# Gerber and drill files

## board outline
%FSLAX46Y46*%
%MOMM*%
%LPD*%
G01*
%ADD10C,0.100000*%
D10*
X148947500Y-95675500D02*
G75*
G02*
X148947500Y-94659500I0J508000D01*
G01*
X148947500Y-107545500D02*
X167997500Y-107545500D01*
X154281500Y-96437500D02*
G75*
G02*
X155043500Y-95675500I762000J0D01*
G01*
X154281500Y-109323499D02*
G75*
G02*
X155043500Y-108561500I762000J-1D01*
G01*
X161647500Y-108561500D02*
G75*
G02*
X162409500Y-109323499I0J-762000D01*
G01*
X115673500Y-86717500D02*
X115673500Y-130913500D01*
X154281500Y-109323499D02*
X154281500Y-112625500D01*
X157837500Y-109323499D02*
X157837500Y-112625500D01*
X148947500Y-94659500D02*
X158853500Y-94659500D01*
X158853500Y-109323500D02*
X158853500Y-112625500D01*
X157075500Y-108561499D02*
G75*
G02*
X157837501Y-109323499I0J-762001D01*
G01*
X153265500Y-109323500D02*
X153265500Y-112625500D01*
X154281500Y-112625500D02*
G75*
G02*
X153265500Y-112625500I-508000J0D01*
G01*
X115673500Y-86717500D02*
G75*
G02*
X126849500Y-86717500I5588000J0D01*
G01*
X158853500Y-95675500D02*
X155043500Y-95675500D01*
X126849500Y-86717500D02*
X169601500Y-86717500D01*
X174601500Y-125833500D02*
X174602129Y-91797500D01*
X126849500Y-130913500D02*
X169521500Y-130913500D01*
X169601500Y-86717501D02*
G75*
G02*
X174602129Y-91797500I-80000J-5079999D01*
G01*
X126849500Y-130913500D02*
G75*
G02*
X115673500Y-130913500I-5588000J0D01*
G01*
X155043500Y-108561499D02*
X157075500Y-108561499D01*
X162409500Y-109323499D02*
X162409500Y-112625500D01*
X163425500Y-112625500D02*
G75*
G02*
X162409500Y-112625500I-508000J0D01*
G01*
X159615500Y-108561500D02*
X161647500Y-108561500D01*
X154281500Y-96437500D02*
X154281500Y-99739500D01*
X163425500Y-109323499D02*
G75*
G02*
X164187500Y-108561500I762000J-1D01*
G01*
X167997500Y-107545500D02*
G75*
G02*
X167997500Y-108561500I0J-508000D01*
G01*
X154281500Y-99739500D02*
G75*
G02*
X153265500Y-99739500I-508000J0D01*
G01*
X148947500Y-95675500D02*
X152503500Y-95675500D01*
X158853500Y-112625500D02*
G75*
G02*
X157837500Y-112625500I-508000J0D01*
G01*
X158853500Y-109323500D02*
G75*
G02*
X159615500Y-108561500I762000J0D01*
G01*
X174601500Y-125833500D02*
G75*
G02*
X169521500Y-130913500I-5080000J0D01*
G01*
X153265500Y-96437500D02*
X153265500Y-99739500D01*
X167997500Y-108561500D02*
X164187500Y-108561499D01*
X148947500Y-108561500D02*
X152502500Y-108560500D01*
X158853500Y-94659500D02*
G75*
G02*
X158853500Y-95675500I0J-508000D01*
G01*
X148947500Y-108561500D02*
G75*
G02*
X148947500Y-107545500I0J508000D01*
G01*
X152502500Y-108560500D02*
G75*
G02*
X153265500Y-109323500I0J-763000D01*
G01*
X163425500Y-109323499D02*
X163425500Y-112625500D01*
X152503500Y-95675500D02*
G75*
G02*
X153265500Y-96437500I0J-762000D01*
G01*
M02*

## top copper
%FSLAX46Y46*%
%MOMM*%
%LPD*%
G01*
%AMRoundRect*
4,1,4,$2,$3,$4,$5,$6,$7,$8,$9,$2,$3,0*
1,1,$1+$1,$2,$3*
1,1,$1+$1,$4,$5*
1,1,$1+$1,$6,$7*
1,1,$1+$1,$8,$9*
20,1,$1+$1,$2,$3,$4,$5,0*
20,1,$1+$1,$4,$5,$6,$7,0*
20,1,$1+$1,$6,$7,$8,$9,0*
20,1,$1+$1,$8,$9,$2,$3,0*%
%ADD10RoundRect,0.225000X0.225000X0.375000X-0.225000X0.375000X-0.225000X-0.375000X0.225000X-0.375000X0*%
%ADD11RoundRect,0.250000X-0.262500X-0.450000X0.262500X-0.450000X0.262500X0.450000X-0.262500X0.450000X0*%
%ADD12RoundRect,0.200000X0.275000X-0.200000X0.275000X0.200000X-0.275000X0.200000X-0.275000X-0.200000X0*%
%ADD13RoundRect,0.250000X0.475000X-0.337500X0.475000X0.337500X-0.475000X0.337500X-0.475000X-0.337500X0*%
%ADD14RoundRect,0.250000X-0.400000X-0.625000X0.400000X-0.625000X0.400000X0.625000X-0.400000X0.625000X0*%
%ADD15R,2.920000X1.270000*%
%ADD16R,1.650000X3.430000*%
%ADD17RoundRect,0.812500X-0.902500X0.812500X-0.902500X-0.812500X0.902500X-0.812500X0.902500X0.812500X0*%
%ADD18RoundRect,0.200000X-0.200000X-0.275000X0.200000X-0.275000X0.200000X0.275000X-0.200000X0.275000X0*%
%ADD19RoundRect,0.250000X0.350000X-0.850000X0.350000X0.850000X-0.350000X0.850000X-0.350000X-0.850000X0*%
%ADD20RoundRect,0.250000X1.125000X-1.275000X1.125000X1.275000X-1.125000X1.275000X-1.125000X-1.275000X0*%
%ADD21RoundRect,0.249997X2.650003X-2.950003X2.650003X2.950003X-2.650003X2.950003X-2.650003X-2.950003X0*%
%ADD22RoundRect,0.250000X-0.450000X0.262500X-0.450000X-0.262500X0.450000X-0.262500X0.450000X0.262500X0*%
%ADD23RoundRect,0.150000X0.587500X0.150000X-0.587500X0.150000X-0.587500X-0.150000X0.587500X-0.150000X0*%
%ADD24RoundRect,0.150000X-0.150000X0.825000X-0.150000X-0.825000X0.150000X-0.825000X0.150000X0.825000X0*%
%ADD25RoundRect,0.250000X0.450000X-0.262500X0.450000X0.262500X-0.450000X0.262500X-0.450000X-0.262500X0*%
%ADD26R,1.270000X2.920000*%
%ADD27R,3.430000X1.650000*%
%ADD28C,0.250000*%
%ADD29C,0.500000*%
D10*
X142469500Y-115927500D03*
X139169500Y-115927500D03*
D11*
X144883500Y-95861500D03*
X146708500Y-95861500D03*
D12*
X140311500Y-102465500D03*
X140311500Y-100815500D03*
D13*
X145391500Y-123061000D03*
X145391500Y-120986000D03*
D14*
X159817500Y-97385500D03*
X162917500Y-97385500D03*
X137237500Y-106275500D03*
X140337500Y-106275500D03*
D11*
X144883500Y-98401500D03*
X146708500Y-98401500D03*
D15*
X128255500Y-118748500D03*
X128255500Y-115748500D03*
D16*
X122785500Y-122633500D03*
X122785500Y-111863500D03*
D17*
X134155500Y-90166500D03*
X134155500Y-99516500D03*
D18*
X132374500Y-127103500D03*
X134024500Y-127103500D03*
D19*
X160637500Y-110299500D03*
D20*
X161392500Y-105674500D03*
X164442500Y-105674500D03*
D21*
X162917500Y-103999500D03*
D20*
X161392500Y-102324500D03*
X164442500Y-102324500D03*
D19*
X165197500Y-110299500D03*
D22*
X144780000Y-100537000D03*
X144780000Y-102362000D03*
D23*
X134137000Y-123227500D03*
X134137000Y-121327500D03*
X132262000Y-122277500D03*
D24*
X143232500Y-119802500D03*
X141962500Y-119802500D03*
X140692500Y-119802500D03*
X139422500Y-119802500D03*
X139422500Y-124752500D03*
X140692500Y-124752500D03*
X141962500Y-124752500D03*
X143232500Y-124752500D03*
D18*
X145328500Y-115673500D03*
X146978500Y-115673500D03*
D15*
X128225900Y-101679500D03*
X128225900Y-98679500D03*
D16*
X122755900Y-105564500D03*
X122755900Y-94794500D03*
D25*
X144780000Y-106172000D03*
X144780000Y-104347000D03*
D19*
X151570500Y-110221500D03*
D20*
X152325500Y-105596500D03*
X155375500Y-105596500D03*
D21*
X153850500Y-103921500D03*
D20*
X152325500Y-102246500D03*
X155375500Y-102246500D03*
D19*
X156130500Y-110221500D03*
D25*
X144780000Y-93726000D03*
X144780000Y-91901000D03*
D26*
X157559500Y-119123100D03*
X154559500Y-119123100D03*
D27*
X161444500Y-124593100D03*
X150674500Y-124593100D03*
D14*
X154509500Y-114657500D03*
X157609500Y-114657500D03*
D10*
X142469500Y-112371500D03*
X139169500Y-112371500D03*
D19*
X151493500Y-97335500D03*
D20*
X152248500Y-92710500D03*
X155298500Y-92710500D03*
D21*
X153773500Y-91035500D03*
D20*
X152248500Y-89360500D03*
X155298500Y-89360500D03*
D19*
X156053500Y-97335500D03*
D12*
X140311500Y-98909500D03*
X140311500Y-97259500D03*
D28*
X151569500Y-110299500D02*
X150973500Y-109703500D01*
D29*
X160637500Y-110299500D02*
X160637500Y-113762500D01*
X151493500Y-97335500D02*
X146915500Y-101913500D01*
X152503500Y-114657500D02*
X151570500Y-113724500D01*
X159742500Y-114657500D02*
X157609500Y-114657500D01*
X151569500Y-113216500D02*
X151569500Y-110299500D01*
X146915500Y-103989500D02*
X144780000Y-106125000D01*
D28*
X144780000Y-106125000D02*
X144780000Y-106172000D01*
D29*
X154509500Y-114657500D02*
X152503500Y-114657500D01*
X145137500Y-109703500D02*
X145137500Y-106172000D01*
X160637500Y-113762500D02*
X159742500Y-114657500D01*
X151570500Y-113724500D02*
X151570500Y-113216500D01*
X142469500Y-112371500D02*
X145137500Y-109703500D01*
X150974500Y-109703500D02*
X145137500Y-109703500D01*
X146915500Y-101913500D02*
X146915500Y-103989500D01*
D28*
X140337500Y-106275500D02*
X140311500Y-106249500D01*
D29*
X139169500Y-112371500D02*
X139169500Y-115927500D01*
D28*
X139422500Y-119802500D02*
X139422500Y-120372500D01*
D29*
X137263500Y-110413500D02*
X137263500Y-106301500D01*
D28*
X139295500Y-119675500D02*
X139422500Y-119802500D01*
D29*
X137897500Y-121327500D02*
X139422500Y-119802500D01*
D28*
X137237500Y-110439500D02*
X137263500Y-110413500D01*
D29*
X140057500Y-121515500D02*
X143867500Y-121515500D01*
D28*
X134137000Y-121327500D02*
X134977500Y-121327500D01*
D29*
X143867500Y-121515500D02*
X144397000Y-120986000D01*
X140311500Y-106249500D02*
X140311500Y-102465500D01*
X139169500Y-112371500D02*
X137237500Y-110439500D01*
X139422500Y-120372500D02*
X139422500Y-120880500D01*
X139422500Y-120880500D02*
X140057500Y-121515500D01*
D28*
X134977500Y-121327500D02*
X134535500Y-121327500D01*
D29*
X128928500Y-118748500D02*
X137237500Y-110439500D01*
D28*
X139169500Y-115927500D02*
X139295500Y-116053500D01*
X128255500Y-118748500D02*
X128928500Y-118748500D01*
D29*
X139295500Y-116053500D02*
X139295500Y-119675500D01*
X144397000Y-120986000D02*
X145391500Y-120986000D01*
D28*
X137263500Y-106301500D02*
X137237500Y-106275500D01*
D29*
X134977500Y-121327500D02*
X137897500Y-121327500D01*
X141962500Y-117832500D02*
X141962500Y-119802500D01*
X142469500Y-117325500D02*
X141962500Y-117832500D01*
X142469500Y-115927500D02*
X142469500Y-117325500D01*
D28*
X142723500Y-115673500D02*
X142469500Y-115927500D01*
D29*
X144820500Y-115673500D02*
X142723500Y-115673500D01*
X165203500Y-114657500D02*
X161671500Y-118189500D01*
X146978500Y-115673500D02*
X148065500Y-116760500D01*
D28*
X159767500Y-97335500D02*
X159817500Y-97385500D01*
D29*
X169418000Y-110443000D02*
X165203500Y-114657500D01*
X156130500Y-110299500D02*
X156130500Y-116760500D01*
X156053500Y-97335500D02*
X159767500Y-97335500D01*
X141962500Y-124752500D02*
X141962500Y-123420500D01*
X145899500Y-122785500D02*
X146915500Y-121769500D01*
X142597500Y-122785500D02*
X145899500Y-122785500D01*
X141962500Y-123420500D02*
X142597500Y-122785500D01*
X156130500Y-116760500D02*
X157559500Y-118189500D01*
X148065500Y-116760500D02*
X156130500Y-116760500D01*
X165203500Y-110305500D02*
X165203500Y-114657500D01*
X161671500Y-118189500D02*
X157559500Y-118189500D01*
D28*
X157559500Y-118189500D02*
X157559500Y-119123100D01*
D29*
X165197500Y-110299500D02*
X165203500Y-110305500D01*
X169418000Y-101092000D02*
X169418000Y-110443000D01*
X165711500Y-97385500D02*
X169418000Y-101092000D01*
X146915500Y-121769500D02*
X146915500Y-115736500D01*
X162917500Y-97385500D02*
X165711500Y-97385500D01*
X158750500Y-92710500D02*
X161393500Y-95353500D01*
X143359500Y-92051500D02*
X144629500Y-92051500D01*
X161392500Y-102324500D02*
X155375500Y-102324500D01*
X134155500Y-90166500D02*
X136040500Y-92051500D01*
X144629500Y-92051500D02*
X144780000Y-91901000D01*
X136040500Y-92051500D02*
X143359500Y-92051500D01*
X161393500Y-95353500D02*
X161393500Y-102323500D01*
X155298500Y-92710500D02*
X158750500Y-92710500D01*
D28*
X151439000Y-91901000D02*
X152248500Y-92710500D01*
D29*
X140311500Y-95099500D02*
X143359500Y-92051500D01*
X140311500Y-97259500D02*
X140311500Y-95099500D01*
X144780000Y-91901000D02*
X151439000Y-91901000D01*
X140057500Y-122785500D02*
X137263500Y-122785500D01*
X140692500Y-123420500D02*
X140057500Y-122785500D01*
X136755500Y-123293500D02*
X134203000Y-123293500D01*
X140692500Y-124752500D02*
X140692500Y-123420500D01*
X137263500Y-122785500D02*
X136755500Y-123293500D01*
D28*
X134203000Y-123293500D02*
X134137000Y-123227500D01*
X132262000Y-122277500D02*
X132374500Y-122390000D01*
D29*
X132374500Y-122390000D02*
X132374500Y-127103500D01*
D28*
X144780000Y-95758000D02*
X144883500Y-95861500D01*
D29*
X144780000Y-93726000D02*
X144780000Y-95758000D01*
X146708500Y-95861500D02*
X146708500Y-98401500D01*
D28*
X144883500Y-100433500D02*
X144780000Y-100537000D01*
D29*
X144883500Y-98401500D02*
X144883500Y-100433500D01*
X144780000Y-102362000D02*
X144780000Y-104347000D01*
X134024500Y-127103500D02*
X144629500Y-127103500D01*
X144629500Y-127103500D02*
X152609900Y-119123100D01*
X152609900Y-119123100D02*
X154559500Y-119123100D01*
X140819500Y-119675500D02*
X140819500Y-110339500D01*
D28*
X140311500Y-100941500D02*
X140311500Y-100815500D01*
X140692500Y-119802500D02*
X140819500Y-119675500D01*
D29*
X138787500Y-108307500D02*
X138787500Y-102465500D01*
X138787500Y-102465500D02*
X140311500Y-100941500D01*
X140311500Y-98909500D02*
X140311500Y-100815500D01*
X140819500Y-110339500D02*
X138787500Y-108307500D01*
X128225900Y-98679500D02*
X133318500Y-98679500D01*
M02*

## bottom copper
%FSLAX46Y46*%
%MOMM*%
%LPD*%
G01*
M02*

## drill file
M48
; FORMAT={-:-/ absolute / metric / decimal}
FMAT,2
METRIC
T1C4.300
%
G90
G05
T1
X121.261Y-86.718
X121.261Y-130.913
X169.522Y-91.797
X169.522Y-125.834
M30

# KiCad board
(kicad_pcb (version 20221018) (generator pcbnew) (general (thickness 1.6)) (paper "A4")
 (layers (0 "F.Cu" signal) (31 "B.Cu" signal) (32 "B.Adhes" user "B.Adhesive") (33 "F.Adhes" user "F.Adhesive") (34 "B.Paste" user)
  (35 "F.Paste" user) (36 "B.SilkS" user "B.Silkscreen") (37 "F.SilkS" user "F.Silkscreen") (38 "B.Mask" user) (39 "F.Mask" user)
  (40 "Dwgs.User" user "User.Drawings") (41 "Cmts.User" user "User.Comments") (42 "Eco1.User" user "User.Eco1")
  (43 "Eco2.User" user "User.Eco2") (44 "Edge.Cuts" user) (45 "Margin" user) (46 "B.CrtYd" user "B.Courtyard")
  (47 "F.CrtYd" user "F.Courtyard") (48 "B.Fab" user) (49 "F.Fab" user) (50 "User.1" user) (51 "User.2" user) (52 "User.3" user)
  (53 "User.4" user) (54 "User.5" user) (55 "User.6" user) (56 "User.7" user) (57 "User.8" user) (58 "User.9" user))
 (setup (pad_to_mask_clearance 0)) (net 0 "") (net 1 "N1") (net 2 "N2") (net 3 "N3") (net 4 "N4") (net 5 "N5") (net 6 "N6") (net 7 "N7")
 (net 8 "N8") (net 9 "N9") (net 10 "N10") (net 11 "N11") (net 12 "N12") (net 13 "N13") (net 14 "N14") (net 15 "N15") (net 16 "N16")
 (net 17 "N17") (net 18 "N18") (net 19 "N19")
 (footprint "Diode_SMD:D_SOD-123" (layer "F.Cu") (at 140.8195 115.9275 180)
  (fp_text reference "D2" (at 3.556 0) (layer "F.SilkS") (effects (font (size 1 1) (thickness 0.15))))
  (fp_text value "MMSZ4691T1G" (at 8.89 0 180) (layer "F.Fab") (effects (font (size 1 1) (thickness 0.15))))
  (pad "1" smd roundrect (at -1.65 0 180) (size 0.9 1.2) (layers "F.Cu" "F.Paste" "F.Mask") (roundrect_rratio 0.25) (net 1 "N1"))
  (pad "2" smd roundrect (at 1.65 0 180) (size 0.9 1.2) (layers "F.Cu" "F.Paste" "F.Mask") (roundrect_rratio 0.25) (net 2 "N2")))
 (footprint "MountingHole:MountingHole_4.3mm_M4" (layer "F.Cu") (at 169.5215 91.7975)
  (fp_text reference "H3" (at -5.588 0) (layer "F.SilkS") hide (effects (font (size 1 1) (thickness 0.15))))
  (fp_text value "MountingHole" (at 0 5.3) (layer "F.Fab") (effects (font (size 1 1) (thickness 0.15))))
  (pad "" np_thru_hole circle (at 0 0) (size 4.3 4.3) (drill 4.3) (layers "*.Cu" "*.Mask")))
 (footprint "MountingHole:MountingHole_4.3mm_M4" (layer "F.Cu") (at 121.2615 130.9135)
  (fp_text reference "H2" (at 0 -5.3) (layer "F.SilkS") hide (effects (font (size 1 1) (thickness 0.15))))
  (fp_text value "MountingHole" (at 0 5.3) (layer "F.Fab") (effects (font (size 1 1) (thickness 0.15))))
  (pad "" np_thru_hole circle (at 0 0) (size 4.3 4.3) (drill 4.3) (layers "*.Cu" "*.Mask")))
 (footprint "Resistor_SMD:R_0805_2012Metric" (layer "F.Cu") (at 145.796 95.8615)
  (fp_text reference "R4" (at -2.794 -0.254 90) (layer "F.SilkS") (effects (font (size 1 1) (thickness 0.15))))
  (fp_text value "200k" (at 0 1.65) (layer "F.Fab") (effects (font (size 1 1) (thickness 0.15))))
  (pad "1" smd roundrect (at -0.9125 0) (size 1.025 1.4) (layers "F.Cu" "F.Paste" "F.Mask") (roundrect_rratio 0.243902) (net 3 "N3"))
  (pad "2" smd roundrect (at 0.9125 0) (size 1.025 1.4) (layers "F.Cu" "F.Paste" "F.Mask") (roundrect_rratio 0.243902) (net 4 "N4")))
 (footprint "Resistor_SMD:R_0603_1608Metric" (layer "F.Cu") (at 140.3115 101.6405 90)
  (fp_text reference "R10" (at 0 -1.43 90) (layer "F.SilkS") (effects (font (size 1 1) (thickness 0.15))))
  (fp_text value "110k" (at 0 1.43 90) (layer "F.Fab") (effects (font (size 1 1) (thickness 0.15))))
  (pad "1" smd roundrect (at -0.825 0 90) (size 0.8 0.95) (layers "F.Cu" "F.Paste" "F.Mask") (roundrect_rratio 0.25) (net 2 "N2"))
  (pad "2" smd roundrect (at 0.825 0 90) (size 0.8 0.95) (layers "F.Cu" "F.Paste" "F.Mask") (roundrect_rratio 0.25) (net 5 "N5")))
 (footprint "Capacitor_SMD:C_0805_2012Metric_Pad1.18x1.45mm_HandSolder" (layer "F.Cu") (at 145.3915 122.0235 90)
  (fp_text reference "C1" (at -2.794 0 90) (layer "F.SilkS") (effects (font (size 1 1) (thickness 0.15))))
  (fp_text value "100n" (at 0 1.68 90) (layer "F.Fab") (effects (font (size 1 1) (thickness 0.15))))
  (pad "1" smd roundrect (at -1.0375 0 90) (size 1.175 1.45) (layers "F.Cu" "F.Paste" "F.Mask") (roundrect_rratio 0.212766) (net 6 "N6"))
  (pad "2" smd roundrect (at 1.0375 0 90) (size 1.175 1.45) (layers "F.Cu" "F.Paste" "F.Mask") (roundrect_rratio 0.212766) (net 2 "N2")))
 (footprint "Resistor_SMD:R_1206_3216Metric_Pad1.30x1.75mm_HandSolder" (layer "F.Cu") (at 161.3675 97.3855)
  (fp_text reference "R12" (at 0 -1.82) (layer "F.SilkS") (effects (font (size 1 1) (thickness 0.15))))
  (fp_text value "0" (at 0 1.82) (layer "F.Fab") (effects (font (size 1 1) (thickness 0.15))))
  (pad "1" smd roundrect (at -1.55 0) (size 1.3 1.75) (layers "F.Cu" "F.Paste" "F.Mask") (roundrect_rratio 0.192308) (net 6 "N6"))
  (pad "2" smd roundrect (at 1.55 0) (size 1.3 1.75) (layers "F.Cu" "F.Paste" "F.Mask") (roundrect_rratio 0.192308) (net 6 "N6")))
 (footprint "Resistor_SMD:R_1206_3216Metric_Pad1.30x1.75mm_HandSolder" (layer "F.Cu") (at 138.7875 106.2755)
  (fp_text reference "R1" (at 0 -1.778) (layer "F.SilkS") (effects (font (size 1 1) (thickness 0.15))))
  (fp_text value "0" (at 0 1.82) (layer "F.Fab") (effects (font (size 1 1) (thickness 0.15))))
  (pad "1" smd roundrect (at -1.55 0) (size 1.3 1.75) (layers "F.Cu" "F.Paste" "F.Mask") (roundrect_rratio 0.192308) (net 2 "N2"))
  (pad "2" smd roundrect (at 1.55 0) (size 1.3 1.75) (layers "F.Cu" "F.Paste" "F.Mask") (roundrect_rratio 0.192308) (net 2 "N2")))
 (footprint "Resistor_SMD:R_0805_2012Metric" (layer "F.Cu") (at 145.796 98.4015)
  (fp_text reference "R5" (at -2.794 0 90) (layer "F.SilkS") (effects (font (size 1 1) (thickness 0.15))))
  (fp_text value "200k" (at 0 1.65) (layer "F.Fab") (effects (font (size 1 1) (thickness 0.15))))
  (pad "1" smd roundrect (at -0.9125 0) (size 1.025 1.4) (layers "F.Cu" "F.Paste" "F.Mask") (roundrect_rratio 0.243902) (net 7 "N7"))
  (pad "2" smd roundrect (at 0.9125 0) (size 1.025 1.4) (layers "F.Cu" "F.Paste" "F.Mask") (roundrect_rratio 0.243902) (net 4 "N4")))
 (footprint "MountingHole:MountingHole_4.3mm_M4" (layer "F.Cu") (at 169.5215 125.8335)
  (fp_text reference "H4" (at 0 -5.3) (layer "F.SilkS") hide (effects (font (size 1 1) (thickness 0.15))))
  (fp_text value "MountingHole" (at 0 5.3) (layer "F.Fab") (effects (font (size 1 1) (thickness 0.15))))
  (pad "" np_thru_hole circle (at 0 0) (size 4.3 4.3) (drill 4.3) (layers "*.Cu" "*.Mask")))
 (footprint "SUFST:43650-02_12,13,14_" (layer "F.Cu") (at 128.2555 117.2485 -90)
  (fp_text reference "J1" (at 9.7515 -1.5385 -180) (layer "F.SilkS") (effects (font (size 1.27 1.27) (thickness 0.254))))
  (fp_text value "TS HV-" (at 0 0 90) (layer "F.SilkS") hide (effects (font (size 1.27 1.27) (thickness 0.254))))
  (pad "1" smd rect (at 1.5 0 270) (size 1.27 2.92) (layers "F.Cu" "F.Paste" "F.Mask") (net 2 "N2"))
  (pad "2" smd rect (at -1.5 0 270) (size 1.27 2.92) (layers "F.Cu" "F.Paste" "F.Mask") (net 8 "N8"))
  (pad "3" smd rect (at 5.385 5.47) (size 1.65 3.43) (layers "F.Cu" "F.Paste" "F.Mask"))
  (pad "4" smd rect (at -5.385 5.47) (size 1.65 3.43) (layers "F.Cu" "F.Paste" "F.Mask")))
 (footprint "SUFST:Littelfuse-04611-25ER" (layer "F.Cu") (at 134.2155 94.5915 -90)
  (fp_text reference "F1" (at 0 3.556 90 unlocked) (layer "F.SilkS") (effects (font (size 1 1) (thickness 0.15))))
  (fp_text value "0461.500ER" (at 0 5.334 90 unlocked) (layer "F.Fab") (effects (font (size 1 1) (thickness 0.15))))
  (pad "1" smd roundrect (at -4.425 0.06 270) (size 3.25 3.43) (layers "F.Cu" "F.Paste" "F.Mask") (roundrect_rratio 0.25) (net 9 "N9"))
  (pad "2" smd roundrect (at 4.925 0.06 270) (size 3.25 3.43) (layers "F.Cu" "F.Paste" "F.Mask") (roundrect_rratio 0.25) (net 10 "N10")))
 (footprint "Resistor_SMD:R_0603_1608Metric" (layer "F.Cu") (at 133.1995 127.1035)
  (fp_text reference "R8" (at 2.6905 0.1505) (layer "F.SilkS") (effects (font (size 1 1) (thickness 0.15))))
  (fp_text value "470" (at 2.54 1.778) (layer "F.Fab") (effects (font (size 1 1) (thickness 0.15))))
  (pad "1" smd roundrect (at -0.825 0) (size 0.8 0.95) (layers "F.Cu" "F.Paste" "F.Mask") (roundrect_rratio 0.25) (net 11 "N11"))
  (pad "2" smd roundrect (at 0.825 0) (size 0.8 0.95) (layers "F.Cu" "F.Paste" "F.Mask") (roundrect_rratio 0.25) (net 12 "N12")))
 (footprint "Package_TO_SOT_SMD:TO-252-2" (layer "F.Cu") (at 162.9175 105.2595 90)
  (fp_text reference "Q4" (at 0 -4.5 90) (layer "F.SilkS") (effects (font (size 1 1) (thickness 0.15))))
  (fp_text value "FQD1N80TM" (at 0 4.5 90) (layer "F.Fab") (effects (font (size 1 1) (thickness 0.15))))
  (pad "1" smd roundrect (at -5.04 -2.28 90) (size 2.2 1.2) (layers "F.Cu" "F.Paste" "F.Mask") (roundrect_rratio 0.208333) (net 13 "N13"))
  (pad "2" smd roundrect (at -0.415 -1.525 90) (size 3.05 2.75) (layers "F.Cu" "F.Paste") (roundrect_rratio 0.090909) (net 9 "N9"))
  (pad "2" smd roundrect (at -0.415 1.525 90) (size 3.05 2.75) (layers "F.Cu" "F.Paste") (roundrect_rratio 0.090909) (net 9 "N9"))
  (pad "2" smd roundrect (at 1.26 0 90) (size 6.4 5.8) (layers "F.Cu" "F.Mask") (roundrect_rratio 0.043103) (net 9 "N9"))
  (pad "2" smd roundrect (at 2.935 -1.525 90) (size 3.05 2.75) (layers "F.Cu" "F.Paste") (roundrect_rratio 0.090909) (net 9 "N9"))
  (pad "2" smd roundrect (at 2.935 1.525 90) (size 3.05 2.75) (layers "F.Cu" "F.Paste") (roundrect_rratio 0.090909) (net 9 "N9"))
  (pad "3" smd roundrect (at -5.04 2.28 90) (size 2.2 1.2) (layers "F.Cu" "F.Paste" "F.Mask") (roundrect_rratio 0.208333) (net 6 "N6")))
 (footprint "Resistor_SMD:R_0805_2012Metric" (layer "F.Cu") (at 144.78 101.4495 -90)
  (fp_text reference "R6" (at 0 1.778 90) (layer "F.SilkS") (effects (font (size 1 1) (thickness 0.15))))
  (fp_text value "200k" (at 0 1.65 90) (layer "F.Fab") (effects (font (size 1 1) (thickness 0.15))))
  (pad "1" smd roundrect (at -0.9125 0 270) (size 1.025 1.4) (layers "F.Cu" "F.Paste" "F.Mask") (roundrect_rratio 0.243902) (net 7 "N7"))
  (pad "2" smd roundrect (at 0.9125 0 270) (size 1.025 1.4) (layers "F.Cu" "F.Paste" "F.Mask") (roundrect_rratio 0.243902) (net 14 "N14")))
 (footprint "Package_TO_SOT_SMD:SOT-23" (layer "F.Cu") (at 133.1995 122.2775 180)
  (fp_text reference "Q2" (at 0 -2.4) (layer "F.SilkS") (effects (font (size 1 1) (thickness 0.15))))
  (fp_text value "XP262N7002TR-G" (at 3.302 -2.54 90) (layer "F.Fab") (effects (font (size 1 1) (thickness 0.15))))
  (pad "1" smd roundrect (at -0.9375 -0.95 180) (size 1.475 0.6) (layers "F.Cu" "F.Paste" "F.Mask") (roundrect_rratio 0.25) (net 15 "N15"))
  (pad "2" smd roundrect (at -0.9375 0.95 180) (size 1.475 0.6) (layers "F.Cu" "F.Paste" "F.Mask") (roundrect_rratio 0.25) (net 2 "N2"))
  (pad "3" smd roundrect (at 0.9375 0 180) (size 1.475 0.6) (layers "F.Cu" "F.Paste" "F.Mask") (roundrect_rratio 0.25) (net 11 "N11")))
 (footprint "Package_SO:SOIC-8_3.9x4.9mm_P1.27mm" (layer "F.Cu") (at 141.3275 122.2775 -90)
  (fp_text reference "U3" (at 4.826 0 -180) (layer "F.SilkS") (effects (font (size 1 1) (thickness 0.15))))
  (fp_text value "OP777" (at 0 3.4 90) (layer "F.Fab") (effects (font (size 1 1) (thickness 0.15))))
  (pad "1" smd roundrect (at -2.475 -1.905 270) (size 1.95 0.6) (layers "F.Cu" "F.Paste" "F.Mask") (roundrect_rratio 0.25) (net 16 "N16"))
  (pad "2" smd roundrect (at -2.475 -0.635 270) (size 1.95 0.6) (layers "F.Cu" "F.Paste" "F.Mask") (roundrect_rratio 0.25) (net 1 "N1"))
  (pad "3" smd roundrect (at -2.475 0.635 270) (size 1.95 0.6) (layers "F.Cu" "F.Paste" "F.Mask") (roundrect_rratio 0.25) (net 5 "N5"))
  (pad "4" smd roundrect (at -2.475 1.905 270) (size 1.95 0.6) (layers "F.Cu" "F.Paste" "F.Mask") (roundrect_rratio 0.25) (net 2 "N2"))
  (pad "5" smd roundrect (at 2.475 1.905 270) (size 1.95 0.6) (layers "F.Cu" "F.Paste" "F.Mask") (roundrect_rratio 0.25) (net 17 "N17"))
  (pad "6" smd roundrect (at 2.475 0.635 270) (size 1.95 0.6) (layers "F.Cu" "F.Paste" "F.Mask") (roundrect_rratio 0.25) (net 15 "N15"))
  (pad "7" smd roundrect (at 2.475 -0.635 270) (size 1.95 0.6) (layers "F.Cu" "F.Paste" "F.Mask") (roundrect_rratio 0.25) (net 6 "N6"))
  (pad "8" smd roundrect (at 2.475 -1.905 270) (size 1.95 0.6) (layers "F.Cu" "F.Paste" "F.Mask") (roundrect_rratio 0.25) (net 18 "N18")))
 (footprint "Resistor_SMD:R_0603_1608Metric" (layer "F.Cu") (at 146.1535 115.6735)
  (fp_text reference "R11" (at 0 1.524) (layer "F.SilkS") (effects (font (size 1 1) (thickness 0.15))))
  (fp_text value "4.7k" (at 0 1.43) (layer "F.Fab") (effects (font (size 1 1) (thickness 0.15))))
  (pad "1" smd roundrect (at -0.825 0) (size 0.8 0.95) (layers "F.Cu" "F.Paste" "F.Mask") (roundrect_rratio 0.25) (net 1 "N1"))
  (pad "2" smd roundrect (at 0.825 0) (size 0.8 0.95) (layers "F.Cu" "F.Paste" "F.Mask") (roundrect_rratio 0.25) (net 6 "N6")))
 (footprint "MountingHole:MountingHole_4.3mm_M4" (layer "F.Cu") (at 121.2615 86.7175)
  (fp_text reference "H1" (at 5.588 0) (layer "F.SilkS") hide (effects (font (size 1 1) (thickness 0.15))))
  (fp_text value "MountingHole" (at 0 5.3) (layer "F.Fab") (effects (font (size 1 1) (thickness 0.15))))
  (pad "" np_thru_hole circle (at 0 0) (size 4.3 4.3) (drill 4.3) (layers "*.Cu" "*.Mask")))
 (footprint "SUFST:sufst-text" (layer "F.Cu") (at 170.5375 109.0695 90)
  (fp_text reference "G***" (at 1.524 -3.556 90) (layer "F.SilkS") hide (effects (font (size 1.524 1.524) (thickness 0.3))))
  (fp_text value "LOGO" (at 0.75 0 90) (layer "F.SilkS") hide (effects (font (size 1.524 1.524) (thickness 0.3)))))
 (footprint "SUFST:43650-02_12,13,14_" (layer "F.Cu") (at 128.2259 100.1795 -90)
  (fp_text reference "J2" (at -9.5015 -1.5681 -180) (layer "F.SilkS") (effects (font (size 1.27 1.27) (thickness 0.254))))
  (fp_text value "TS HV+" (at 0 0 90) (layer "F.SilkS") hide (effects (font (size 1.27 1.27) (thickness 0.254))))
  (pad "1" smd rect (at 1.5 0 270) (size 1.27 2.92) (layers "F.Cu" "F.Paste" "F.Mask") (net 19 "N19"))
  (pad "2" smd rect (at -1.5 0 270) (size 1.27 2.92) (layers "F.Cu" "F.Paste" "F.Mask") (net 10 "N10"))
  (pad "3" smd rect (at 5.385 5.47) (size 1.65 3.43) (layers "F.Cu" "F.Paste" "F.Mask"))
  (pad "4" smd rect (at -5.385 5.47) (size 1.65 3.43) (layers "F.Cu" "F.Paste" "F.Mask")))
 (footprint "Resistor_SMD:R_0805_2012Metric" (layer "F.Cu") (at 144.78 105.2595 90)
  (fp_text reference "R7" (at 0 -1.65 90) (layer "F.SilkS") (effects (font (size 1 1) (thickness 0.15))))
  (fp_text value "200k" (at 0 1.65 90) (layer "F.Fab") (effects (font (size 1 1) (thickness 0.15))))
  (pad "1" smd roundrect (at -0.9125 0 90) (size 1.025 1.4) (layers "F.Cu" "F.Paste" "F.Mask") (roundrect_rratio 0.243902) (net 13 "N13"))
  (pad "2" smd roundrect (at 0.9125 0 90) (size 1.025 1.4) (layers "F.Cu" "F.Paste" "F.Mask") (roundrect_rratio 0.243902) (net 14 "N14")))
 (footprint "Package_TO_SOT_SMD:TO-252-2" (layer "F.Cu") (at 153.8505 105.1815 90)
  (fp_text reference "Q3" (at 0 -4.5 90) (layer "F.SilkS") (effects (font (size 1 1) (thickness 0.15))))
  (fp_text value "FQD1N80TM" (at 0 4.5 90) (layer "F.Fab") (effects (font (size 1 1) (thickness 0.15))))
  (pad "1" smd roundrect (at -5.04 -2.28 90) (size 2.2 1.2) (layers "F.Cu" "F.Paste" "F.Mask") (roundrect_rratio 0.208333) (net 13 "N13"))
  (pad "2" smd roundrect (at -0.415 -1.525 90) (size 3.05 2.75) (layers "F.Cu" "F.Paste") (roundrect_rratio 0.090909) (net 9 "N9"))
  (pad "2" smd roundrect (at -0.415 1.525 90) (size 3.05 2.75) (layers "F.Cu" "F.Paste") (roundrect_rratio 0.090909) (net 9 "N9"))
  (pad "2" smd roundrect (at 1.26 0 90) (size 6.4 5.8) (layers "F.Cu" "F.Mask") (roundrect_rratio 0.043103) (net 9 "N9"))
  (pad "2" smd roundrect (at 2.935 -1.525 90) (size 3.05 2.75) (layers "F.Cu" "F.Paste") (roundrect_rratio 0.090909) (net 9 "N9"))
  (pad "2" smd roundrect (at 2.935 1.525 90) (size 3.05 2.75) (layers "F.Cu" "F.Paste") (roundrect_rratio 0.090909) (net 9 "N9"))
  (pad "3" smd roundrect (at -5.04 2.28 90) (size 2.2 1.2) (layers "F.Cu" "F.Paste" "F.Mask") (roundrect_rratio 0.208333) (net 6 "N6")))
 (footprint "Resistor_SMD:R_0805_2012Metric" (layer "F.Cu") (at 144.78 92.8135 90)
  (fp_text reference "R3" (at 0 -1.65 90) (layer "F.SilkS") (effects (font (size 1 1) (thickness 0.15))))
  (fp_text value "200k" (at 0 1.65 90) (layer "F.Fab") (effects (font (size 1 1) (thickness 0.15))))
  (pad "1" smd roundrect (at -0.9125 0 90) (size 1.025 1.4) (layers "F.Cu" "F.Paste" "F.Mask") (roundrect_rratio 0.243902) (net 3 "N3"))
  (pad "2" smd roundrect (at 0.9125 0 90) (size 1.025 1.4) (layers "F.Cu" "F.Paste" "F.Mask") (roundrect_rratio 0.243902) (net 9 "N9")))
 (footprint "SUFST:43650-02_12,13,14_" (layer "F.Cu") (at 156.0595 119.1231)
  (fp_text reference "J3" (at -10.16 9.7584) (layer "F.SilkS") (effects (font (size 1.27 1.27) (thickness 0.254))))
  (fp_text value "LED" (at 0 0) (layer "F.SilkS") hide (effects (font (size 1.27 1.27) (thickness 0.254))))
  (pad "1" smd rect (at 1.5 0) (size 1.27 2.92) (layers "F.Cu" "F.Paste" "F.Mask") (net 6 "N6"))
  (pad "2" smd rect (at -1.5 0) (size 1.27 2.92) (layers "F.Cu" "F.Paste" "F.Mask") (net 12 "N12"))
  (pad "3" smd rect (at 5.385 5.47 90) (size 1.65 3.43) (layers "F.Cu" "F.Paste" "F.Mask"))
  (pad "4" smd rect (at -5.385 5.47 90) (size 1.65 3.43) (layers "F.Cu" "F.Paste" "F.Mask")))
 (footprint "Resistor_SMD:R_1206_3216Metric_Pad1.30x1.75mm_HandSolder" (layer "F.Cu") (at 156.0595 114.6575)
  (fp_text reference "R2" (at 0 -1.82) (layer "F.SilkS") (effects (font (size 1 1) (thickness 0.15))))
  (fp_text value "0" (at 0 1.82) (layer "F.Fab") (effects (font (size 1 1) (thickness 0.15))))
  (pad "1" smd roundrect (at -1.55 0) (size 1.3 1.75) (layers "F.Cu" "F.Paste" "F.Mask") (roundrect_rratio 0.192308) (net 13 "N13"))
  (pad "2" smd roundrect (at 1.55 0) (size 1.3 1.75) (layers "F.Cu" "F.Paste" "F.Mask") (roundrect_rratio 0.192308) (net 13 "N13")))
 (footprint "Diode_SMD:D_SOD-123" (layer "F.Cu") (at 140.8195 112.3715 180)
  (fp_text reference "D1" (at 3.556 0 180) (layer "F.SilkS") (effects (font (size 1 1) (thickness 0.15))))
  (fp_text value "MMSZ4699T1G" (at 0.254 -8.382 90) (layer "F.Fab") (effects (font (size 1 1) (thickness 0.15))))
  (pad "1" smd roundrect (at -1.65 0 180) (size 0.9 1.2) (layers "F.Cu" "F.Paste" "F.Mask") (roundrect_rratio 0.25) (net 13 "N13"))
  (pad "2" smd roundrect (at 1.65 0 180) (size 0.9 1.2) (layers "F.Cu" "F.Paste" "F.Mask") (roundrect_rratio 0.25) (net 2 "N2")))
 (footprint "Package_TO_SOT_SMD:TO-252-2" (layer "F.Cu") (at 153.7735 92.2955 90)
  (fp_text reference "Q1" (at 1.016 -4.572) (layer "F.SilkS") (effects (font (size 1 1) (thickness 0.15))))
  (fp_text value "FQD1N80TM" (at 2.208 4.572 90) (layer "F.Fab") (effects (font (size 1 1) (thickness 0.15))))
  (pad "1" smd roundrect (at -5.04 -2.28 90) (size 2.2 1.2) (layers "F.Cu" "F.Paste" "F.Mask") (roundrect_rratio 0.208333) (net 13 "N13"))
  (pad "2" smd roundrect (at -0.415 -1.525 90) (size 3.05 2.75) (layers "F.Cu" "F.Paste") (roundrect_rratio 0.090909) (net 9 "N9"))
  (pad "2" smd roundrect (at -0.415 1.525 90) (size 3.05 2.75) (layers "F.Cu" "F.Paste") (roundrect_rratio 0.090909) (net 9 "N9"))
  (pad "2" smd roundrect (at 1.26 0 90) (size 6.4 5.8) (layers "F.Cu" "F.Mask") (roundrect_rratio 0.043103) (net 9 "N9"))
  (pad "2" smd roundrect (at 2.935 -1.525 90) (size 3.05 2.75) (layers "F.Cu" "F.Paste") (roundrect_rratio 0.090909) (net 9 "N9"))
  (pad "2" smd roundrect (at 2.935 1.525 90) (size 3.05 2.75) (layers "F.Cu" "F.Paste") (roundrect_rratio 0.090909) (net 9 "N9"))
  (pad "3" smd roundrect (at -5.04 2.28 90) (size 2.2 1.2) (layers "F.Cu" "F.Paste" "F.Mask") (roundrect_rratio 0.208333) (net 6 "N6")))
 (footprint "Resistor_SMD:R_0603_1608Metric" (layer "F.Cu") (at 140.3115 98.0845 90)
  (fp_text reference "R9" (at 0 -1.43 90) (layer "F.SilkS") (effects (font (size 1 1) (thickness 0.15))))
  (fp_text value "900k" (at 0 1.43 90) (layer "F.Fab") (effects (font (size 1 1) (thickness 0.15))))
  (pad "1" smd roundrect (at -0.825 0 90) (size 0.8 0.95) (layers "F.Cu" "F.Paste" "F.Mask") (roundrect_rratio 0.25) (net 5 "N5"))
  (pad "2" smd roundrect (at 0.825 0 90) (size 0.8 0.95) (layers "F.Cu" "F.Paste" "F.Mask") (roundrect_rratio 0.25) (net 9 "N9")))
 (gr_arc (start 148.9475 95.6755) (mid 148.4395 95.1675) (end 148.9475 94.6595) (stroke (width 0.1) (type default)) (layer "Edge.Cuts"))
 (gr_line (start 148.9475 107.5455) (end 167.9975 107.5455) (stroke (width 0.1) (type default)) (layer "Edge.Cuts"))
 (gr_arc (start 154.2815 96.4375) (mid 154.504685 95.898685) (end 155.0435 95.6755) (stroke (width 0.1) (type default)) (layer "Edge.Cuts"))
 (gr_arc (start 154.2815 109.323499) (mid 154.504685 108.784684) (end 155.0435 108.561499) (stroke (width 0.1) (type default))
  (layer "Edge.Cuts"))
 (gr_arc (start 161.6475 108.5615) (mid 162.186315 108.784684) (end 162.4095 109.323499) (stroke (width 0.1) (type default))
  (layer "Edge.Cuts"))
 (gr_line (start 115.6735 86.7175) (end 115.6735 130.9135) (stroke (width 0.1) (type default)) (layer "Edge.Cuts"))
 (gr_line (start 154.2815 109.323499) (end 154.2815 112.6255) (stroke (width 0.1) (type default)) (layer "Edge.Cuts"))
 (gr_line (start 157.8375 109.323499) (end 157.8375 112.6255) (stroke (width 0.1) (type default)) (layer "Edge.Cuts"))
 (gr_line (start 148.9475 94.6595) (end 158.8535 94.6595) (stroke (width 0.1) (type default)) (layer "Edge.Cuts"))
 (gr_line (start 158.8535 109.3235) (end 158.8535 112.6255) (stroke (width 0.1) (type default)) (layer "Edge.Cuts"))
 (gr_arc (start 157.0755 108.561499) (mid 157.614315 108.784684) (end 157.8375 109.323499) (stroke (width 0.1) (type default))
  (layer "Edge.Cuts"))
 (gr_line (start 153.2655 109.3235) (end 153.2655 112.6255) (stroke (width 0.1) (type default)) (layer "Edge.Cuts"))
 (gr_arc (start 154.2815 112.6255) (mid 153.7735 113.1335) (end 153.2655 112.6255) (stroke (width 0.1) (type default)) (layer "Edge.Cuts"))
 (gr_arc (start 115.6735 86.7175) (mid 121.2615 81.1295) (end 126.8495 86.7175) (stroke (width 0.1) (type default)) (layer "Edge.Cuts"))
 (gr_line (start 158.8535 95.6755) (end 155.0435 95.6755) (stroke (width 0.1) (type default)) (layer "Edge.Cuts"))
 (gr_line (start 126.8495 86.7175) (end 169.6015 86.7175) (stroke (width 0.1) (type default)) (layer "Edge.Cuts"))
 (gr_line (start 174.6015 125.8335) (end 174.602129 91.7975) (stroke (width 0.1) (type default)) (layer "Edge.Cuts"))
 (gr_line (start 126.8495 130.9135) (end 169.5215 130.9135) (stroke (width 0.1) (type default)) (layer "Edge.Cuts"))
 (gr_arc (start 169.6015 86.717501) (mid 173.142221 88.233349) (end 174.602129 91.7975) (stroke (width 0.1) (type default))
  (layer "Edge.Cuts"))
 (gr_arc (start 126.8495 130.9135) (mid 121.2615 136.5015) (end 115.6735 130.9135) (stroke (width 0.1) (type default)) (layer "Edge.Cuts"))
 (gr_line (start 155.0435 108.561499) (end 157.0755 108.561499) (stroke (width 0.1) (type default)) (layer "Edge.Cuts"))
 (gr_line (start 162.4095 109.323499) (end 162.4095 112.6255) (stroke (width 0.1) (type default)) (layer "Edge.Cuts"))
 (gr_arc (start 163.4255 112.6255) (mid 162.9175 113.1335) (end 162.4095 112.6255) (stroke (width 0.1) (type default)) (layer "Edge.Cuts"))
 (gr_line (start 159.6155 108.5615) (end 161.6475 108.5615) (stroke (width 0.1) (type default)) (layer "Edge.Cuts"))
 (gr_line (start 154.2815 96.4375) (end 154.2815 99.7395) (stroke (width 0.1) (type default)) (layer "Edge.Cuts"))
 (gr_arc (start 163.4255 109.323499) (mid 163.648685 108.784684) (end 164.1875 108.561499) (stroke (width 0.1) (type default))
  (layer "Edge.Cuts"))
 (gr_arc (start 167.9975 107.5455) (mid 168.5055 108.0535) (end 167.9975 108.5615) (stroke (width 0.1) (type default)) (layer "Edge.Cuts"))
 (gr_arc (start 154.2815 99.7395) (mid 153.7735 100.2475) (end 153.2655 99.7395) (stroke (width 0.1) (type default)) (layer "Edge.Cuts"))
 (gr_line (start 148.9475 95.6755) (end 152.5035 95.6755) (stroke (width 0.1) (type default)) (layer "Edge.Cuts"))
 (gr_arc (start 158.8535 112.6255) (mid 158.3455 113.1335) (end 157.8375 112.6255) (stroke (width 0.1) (type default)) (layer "Edge.Cuts"))
 (gr_arc (start 158.8535 109.3235) (mid 159.076685 108.784685) (end 159.6155 108.5615) (stroke (width 0.1) (type default))
  (layer "Edge.Cuts"))
 (gr_arc (start 174.6015 125.8335) (mid 173.113602 129.425602) (end 169.5215 130.9135) (stroke (width 0.1) (type default))
  (layer "Edge.Cuts"))
 (gr_line (start 153.2655 96.4375) (end 153.2655 99.7395) (stroke (width 0.1) (type default)) (layer "Edge.Cuts"))
 (gr_line (start 167.9975 108.5615) (end 164.1875 108.561499) (stroke (width 0.1) (type default)) (layer "Edge.Cuts"))
 (gr_line (start 148.9475 108.5615) (end 152.5025 108.5605) (stroke (width 0.1) (type default)) (layer "Edge.Cuts"))
 (gr_arc (start 158.8535 94.6595) (mid 159.3615 95.1675) (end 158.8535 95.6755) (stroke (width 0.1) (type default)) (layer "Edge.Cuts"))
 (gr_arc (start 148.9475 108.5615) (mid 148.4395 108.0535) (end 148.9475 107.5455) (stroke (width 0.1) (type default)) (layer "Edge.Cuts"))
 (gr_arc (start 152.5025 108.5605) (mid 153.042022 108.783978) (end 153.2655 109.3235) (stroke (width 0.1) (type default))
  (layer "Edge.Cuts"))
 (gr_line (start 163.4255 109.323499) (end 163.4255 112.6255) (stroke (width 0.1) (type default)) (layer "Edge.Cuts"))
 (gr_arc (start 152.5035 95.6755) (mid 153.042315 95.898685) (end 153.2655 96.4375) (stroke (width 0.1) (type default)) (layer "Edge.Cuts"))
 (segment (start 151.5695 110.2995) (end 150.9735 109.7035) (width 0.25) (layer "F.Cu") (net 13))
 (segment (start 160.6375 110.2995) (end 160.6375 113.7625) (width 0.5) (layer "F.Cu") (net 13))
 (segment (start 151.4935 97.3355) (end 146.9155 101.9135) (width 0.5) (layer "F.Cu") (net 13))
 (segment (start 152.5035 114.6575) (end 151.5705 113.7245) (width 0.5) (layer "F.Cu") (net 13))
 (segment (start 159.7425 114.6575) (end 157.6095 114.6575) (width 0.5) (layer "F.Cu") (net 13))
 (segment (start 151.5695 113.2165) (end 151.5695 110.2995) (width 0.5) (layer "F.Cu") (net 13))
 (segment (start 146.9155 103.9895) (end 144.78 106.125) (width 0.5) (layer "F.Cu") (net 13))
 (segment (start 144.78 106.125) (end 144.78 106.172) (width 0.25) (layer "F.Cu") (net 13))
 (segment (start 154.5095 114.6575) (end 152.5035 114.6575) (width 0.5) (layer "F.Cu") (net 13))
 (segment (start 145.1375 109.7035) (end 145.1375 106.172) (width 0.5) (layer "F.Cu") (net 13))
 (segment (start 160.6375 113.7625) (end 159.7425 114.6575) (width 0.5) (layer "F.Cu") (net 13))
 (segment (start 151.5705 113.7245) (end 151.5705 113.2165) (width 0.5) (layer "F.Cu") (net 13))
 (segment (start 142.4695 112.3715) (end 145.1375 109.7035) (width 0.5) (layer "F.Cu") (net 13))
 (segment (start 150.9745 109.7035) (end 145.1375 109.7035) (width 0.5) (layer "F.Cu") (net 13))
 (segment (start 146.9155 101.9135) (end 146.9155 103.9895) (width 0.5) (layer "F.Cu") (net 13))
 (segment (start 140.3375 106.2755) (end 140.3115 106.2495) (width 0.25) (layer "F.Cu") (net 2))
 (segment (start 139.1695 112.3715) (end 139.1695 115.9275) (width 0.5) (layer "F.Cu") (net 2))
 (segment (start 139.4225 119.8025) (end 139.4225 120.3725) (width 0.25) (layer "F.Cu") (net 2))
 (segment (start 137.2635 110.4135) (end 137.2635 106.3015) (width 0.5) (layer "F.Cu") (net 2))
 (segment (start 139.2955 119.6755) (end 139.4225 119.8025) (width 0.25) (layer "F.Cu") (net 2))
 (segment (start 137.8975 121.3275) (end 139.4225 119.8025) (width 0.5) (layer "F.Cu") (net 2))
 (segment (start 137.2375 110.4395) (end 137.2635 110.4135) (width 0.25) (layer "F.Cu") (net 2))
 (segment (start 140.0575 121.5155) (end 143.8675 121.5155) (width 0.5) (layer "F.Cu") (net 2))
 (segment (start 134.137 121.3275) (end 134.9775 121.3275) (width 0.25) (layer "F.Cu") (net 2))
 (segment (start 143.8675 121.5155) (end 144.397 120.986) (width 0.5) (layer "F.Cu") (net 2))
 (segment (start 140.3115 106.2495) (end 140.3115 102.4655) (width 0.5) (layer "F.Cu") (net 2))
 (segment (start 139.1695 112.3715) (end 137.2375 110.4395) (width 0.5) (layer "F.Cu") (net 2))
 (segment (start 139.4225 120.3725) (end 139.4225 120.8805) (width 0.5) (layer "F.Cu") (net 2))
 (segment (start 139.4225 120.8805) (end 140.0575 121.5155) (width 0.5) (layer "F.Cu") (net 2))
 (segment (start 134.9775 121.3275) (end 134.5355 121.3275) (width 0.25) (layer "F.Cu") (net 2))
 (segment (start 128.9285 118.7485) (end 137.2375 110.4395) (width 0.5) (layer "F.Cu") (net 2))
 (segment (start 139.1695 115.9275) (end 139.2955 116.0535) (width 0.25) (layer "F.Cu") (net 2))
 (segment (start 128.2555 118.7485) (end 128.9285 118.7485) (width 0.25) (layer "F.Cu") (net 2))
 (segment (start 139.2955 116.0535) (end 139.2955 119.6755) (width 0.5) (layer "F.Cu") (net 2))
 (segment (start 144.397 120.986) (end 145.3915 120.986) (width 0.5) (layer "F.Cu") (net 2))
 (segment (start 137.2635 106.3015) (end 137.2375 106.2755) (width 0.25) (layer "F.Cu") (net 2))
 (segment (start 134.9775 121.3275) (end 137.8975 121.3275) (width 0.5) (layer "F.Cu") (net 2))
 (segment (start 141.9625 117.8325) (end 141.9625 119.8025) (width 0.5) (layer "F.Cu") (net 1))
 (segment (start 142.4695 117.3255) (end 141.9625 117.8325) (width 0.5) (layer "F.Cu") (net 1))
 (segment (start 142.4695 115.9275) (end 142.4695 117.3255) (width 0.5) (layer "F.Cu") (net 1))
 (segment (start 142.7235 115.6735) (end 142.4695 115.9275) (width 0.25) (layer "F.Cu") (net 1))
 (segment (start 144.8205 115.6735) (end 142.7235 115.6735) (width 0.5) (layer "F.Cu") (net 1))
 (segment (start 165.2035 114.6575) (end 161.6715 118.1895) (width 0.5) (layer "F.Cu") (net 6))
 (segment (start 146.9785 115.6735) (end 148.0655 116.7605) (width 0.5) (layer "F.Cu") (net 6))
 (segment (start 159.7675 97.3355) (end 159.8175 97.3855) (width 0.25) (layer "F.Cu") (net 6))
 (segment (start 169.418 110.443) (end 165.2035 114.6575) (width 0.5) (layer "F.Cu") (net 6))
 (segment (start 156.1305 110.2995) (end 156.1305 116.7605) (width 0.5) (layer "F.Cu") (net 6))
 (segment (start 156.0535 97.3355) (end 159.7675 97.3355) (width 0.5) (layer "F.Cu") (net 6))
 (segment (start 141.9625 124.7525) (end 141.9625 123.4205) (width 0.5) (layer "F.Cu") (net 6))
 (segment (start 145.8995 122.7855) (end 146.9155 121.7695) (width 0.5) (layer "F.Cu") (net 6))
 (segment (start 142.5975 122.7855) (end 145.8995 122.7855) (width 0.5) (layer "F.Cu") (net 6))
 (segment (start 141.9625 123.4205) (end 142.5975 122.7855) (width 0.5) (layer "F.Cu") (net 6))
 (segment (start 156.1305 116.7605) (end 157.5595 118.1895) (width 0.5) (layer "F.Cu") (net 6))
 (segment (start 148.0655 116.7605) (end 156.1305 116.7605) (width 0.5) (layer "F.Cu") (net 6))
 (segment (start 165.2035 110.3055) (end 165.2035 114.6575) (width 0.5) (layer "F.Cu") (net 6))
 (segment (start 161.6715 118.1895) (end 157.5595 118.1895) (width 0.5) (layer "F.Cu") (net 6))
 (segment (start 157.5595 118.1895) (end 157.5595 119.1231) (width 0.25) (layer "F.Cu") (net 6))
 (segment (start 165.1975 110.2995) (end 165.2035 110.3055) (width 0.5) (layer "F.Cu") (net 6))
 (segment (start 169.418 101.092) (end 169.418 110.443) (width 0.5) (layer "F.Cu") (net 6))
 (segment (start 165.7115 97.3855) (end 169.418 101.092) (width 0.5) (layer "F.Cu") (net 6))
 (segment (start 146.9155 121.7695) (end 146.9155 115.7365) (width 0.5) (layer "F.Cu") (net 6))
 (segment (start 162.9175 97.3855) (end 165.7115 97.3855) (width 0.5) (layer "F.Cu") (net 6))
 (segment (start 158.7505 92.7105) (end 161.3935 95.3535) (width 0.5) (layer "F.Cu") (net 9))
 (segment (start 143.3595 92.0515) (end 144.6295 92.0515) (width 0.5) (layer "F.Cu") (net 9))
 (segment (start 161.3925 102.3245) (end 155.3755 102.3245) (width 0.5) (layer "F.Cu") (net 9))
 (segment (start 134.1555 90.1665) (end 136.0405 92.0515) (width 0.5) (layer "F.Cu") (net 9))
 (segment (start 144.6295 92.0515) (end 144.78 91.901) (width 0.5) (layer "F.Cu") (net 9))
 (segment (start 136.0405 92.0515) (end 143.3595 92.0515) (width 0.5) (layer "F.Cu") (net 9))
 (segment (start 161.3935 95.3535) (end 161.3935 102.3235) (width 0.5) (layer "F.Cu") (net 9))
 (segment (start 155.2985 92.7105) (end 158.7505 92.7105) (width 0.5) (layer "F.Cu") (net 9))
 (segment (start 151.439 91.901) (end 152.2485 92.7105) (width 0.25) (layer "F.Cu") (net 9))
 (segment (start 140.3115 95.0995) (end 143.3595 92.0515) (width 0.5) (layer "F.Cu") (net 9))
 (segment (start 140.3115 97.2595) (end 140.3115 95.0995) (width 0.5) (layer "F.Cu") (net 9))
 (segment (start 144.78 91.901) (end 151.439 91.901) (width 0.5) (layer "F.Cu") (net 9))
 (segment (start 140.0575 122.7855) (end 137.2635 122.7855) (width 0.5) (layer "F.Cu") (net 15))
 (segment (start 140.6925 123.4205) (end 140.0575 122.7855) (width 0.5) (layer "F.Cu") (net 15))
 (segment (start 136.7555 123.2935) (end 134.203 123.2935) (width 0.5) (layer "F.Cu") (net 15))
 (segment (start 140.6925 124.7525) (end 140.6925 123.4205) (width 0.5) (layer "F.Cu") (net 15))
 (segment (start 137.2635 122.7855) (end 136.7555 123.2935) (width 0.5) (layer "F.Cu") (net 15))
 (segment (start 134.203 123.2935) (end 134.137 123.2275) (width 0.25) (layer "F.Cu") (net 15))
 (segment (start 132.262 122.2775) (end 132.3745 122.39) (width 0.25) (layer "F.Cu") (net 11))
 (segment (start 132.3745 122.39) (end 132.3745 127.1035) (width 0.5) (layer "F.Cu") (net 11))
 (segment (start 144.78 95.758) (end 144.8835 95.8615) (width 0.25) (layer "F.Cu") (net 3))
 (segment (start 144.78 93.726) (end 144.78 95.758) (width 0.5) (layer "F.Cu") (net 3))
 (segment (start 146.7085 95.8615) (end 146.7085 98.4015) (width 0.5) (layer "F.Cu") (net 4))
 (segment (start 144.8835 100.4335) (end 144.78 100.537) (width 0.25) (layer "F.Cu") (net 7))
 (segment (start 144.8835 98.4015) (end 144.8835 100.4335) (width 0.5) (layer "F.Cu") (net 7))
 (segment (start 144.78 102.362) (end 144.78 104.347) (width 0.5) (layer "F.Cu") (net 14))
 (segment (start 134.0245 127.1035) (end 144.6295 127.1035) (width 0.5) (layer "F.Cu") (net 12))
 (segment (start 144.6295 127.1035) (end 152.6099 119.1231) (width 0.5) (layer "F.Cu") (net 12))
 (segment (start 152.6099 119.1231) (end 154.5595 119.1231) (width 0.5) (layer "F.Cu") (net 12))
 (segment (start 140.8195 119.6755) (end 140.8195 110.3395) (width 0.5) (layer "F.Cu") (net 5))
 (segment (start 140.3115 100.9415) (end 140.3115 100.8155) (width 0.25) (layer "F.Cu") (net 5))
 (segment (start 140.6925 119.8025) (end 140.8195 119.6755) (width 0.25) (layer "F.Cu") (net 5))
 (segment (start 138.7875 108.3075) (end 138.7875 102.4655) (width 0.5) (layer "F.Cu") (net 5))
 (segment (start 138.7875 102.4655) (end 140.3115 100.9415) (width 0.5) (layer "F.Cu") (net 5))
 (segment (start 140.3115 98.9095) (end 140.3115 100.8155) (width 0.5) (layer "F.Cu") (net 5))
 (segment (start 140.8195 110.3395) (end 138.7875 108.3075) (width 0.5) (layer "F.Cu") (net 5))
 (segment (start 128.2259 98.6795) (end 133.3185 98.6795) (width 0.5) (layer "F.Cu") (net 10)))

